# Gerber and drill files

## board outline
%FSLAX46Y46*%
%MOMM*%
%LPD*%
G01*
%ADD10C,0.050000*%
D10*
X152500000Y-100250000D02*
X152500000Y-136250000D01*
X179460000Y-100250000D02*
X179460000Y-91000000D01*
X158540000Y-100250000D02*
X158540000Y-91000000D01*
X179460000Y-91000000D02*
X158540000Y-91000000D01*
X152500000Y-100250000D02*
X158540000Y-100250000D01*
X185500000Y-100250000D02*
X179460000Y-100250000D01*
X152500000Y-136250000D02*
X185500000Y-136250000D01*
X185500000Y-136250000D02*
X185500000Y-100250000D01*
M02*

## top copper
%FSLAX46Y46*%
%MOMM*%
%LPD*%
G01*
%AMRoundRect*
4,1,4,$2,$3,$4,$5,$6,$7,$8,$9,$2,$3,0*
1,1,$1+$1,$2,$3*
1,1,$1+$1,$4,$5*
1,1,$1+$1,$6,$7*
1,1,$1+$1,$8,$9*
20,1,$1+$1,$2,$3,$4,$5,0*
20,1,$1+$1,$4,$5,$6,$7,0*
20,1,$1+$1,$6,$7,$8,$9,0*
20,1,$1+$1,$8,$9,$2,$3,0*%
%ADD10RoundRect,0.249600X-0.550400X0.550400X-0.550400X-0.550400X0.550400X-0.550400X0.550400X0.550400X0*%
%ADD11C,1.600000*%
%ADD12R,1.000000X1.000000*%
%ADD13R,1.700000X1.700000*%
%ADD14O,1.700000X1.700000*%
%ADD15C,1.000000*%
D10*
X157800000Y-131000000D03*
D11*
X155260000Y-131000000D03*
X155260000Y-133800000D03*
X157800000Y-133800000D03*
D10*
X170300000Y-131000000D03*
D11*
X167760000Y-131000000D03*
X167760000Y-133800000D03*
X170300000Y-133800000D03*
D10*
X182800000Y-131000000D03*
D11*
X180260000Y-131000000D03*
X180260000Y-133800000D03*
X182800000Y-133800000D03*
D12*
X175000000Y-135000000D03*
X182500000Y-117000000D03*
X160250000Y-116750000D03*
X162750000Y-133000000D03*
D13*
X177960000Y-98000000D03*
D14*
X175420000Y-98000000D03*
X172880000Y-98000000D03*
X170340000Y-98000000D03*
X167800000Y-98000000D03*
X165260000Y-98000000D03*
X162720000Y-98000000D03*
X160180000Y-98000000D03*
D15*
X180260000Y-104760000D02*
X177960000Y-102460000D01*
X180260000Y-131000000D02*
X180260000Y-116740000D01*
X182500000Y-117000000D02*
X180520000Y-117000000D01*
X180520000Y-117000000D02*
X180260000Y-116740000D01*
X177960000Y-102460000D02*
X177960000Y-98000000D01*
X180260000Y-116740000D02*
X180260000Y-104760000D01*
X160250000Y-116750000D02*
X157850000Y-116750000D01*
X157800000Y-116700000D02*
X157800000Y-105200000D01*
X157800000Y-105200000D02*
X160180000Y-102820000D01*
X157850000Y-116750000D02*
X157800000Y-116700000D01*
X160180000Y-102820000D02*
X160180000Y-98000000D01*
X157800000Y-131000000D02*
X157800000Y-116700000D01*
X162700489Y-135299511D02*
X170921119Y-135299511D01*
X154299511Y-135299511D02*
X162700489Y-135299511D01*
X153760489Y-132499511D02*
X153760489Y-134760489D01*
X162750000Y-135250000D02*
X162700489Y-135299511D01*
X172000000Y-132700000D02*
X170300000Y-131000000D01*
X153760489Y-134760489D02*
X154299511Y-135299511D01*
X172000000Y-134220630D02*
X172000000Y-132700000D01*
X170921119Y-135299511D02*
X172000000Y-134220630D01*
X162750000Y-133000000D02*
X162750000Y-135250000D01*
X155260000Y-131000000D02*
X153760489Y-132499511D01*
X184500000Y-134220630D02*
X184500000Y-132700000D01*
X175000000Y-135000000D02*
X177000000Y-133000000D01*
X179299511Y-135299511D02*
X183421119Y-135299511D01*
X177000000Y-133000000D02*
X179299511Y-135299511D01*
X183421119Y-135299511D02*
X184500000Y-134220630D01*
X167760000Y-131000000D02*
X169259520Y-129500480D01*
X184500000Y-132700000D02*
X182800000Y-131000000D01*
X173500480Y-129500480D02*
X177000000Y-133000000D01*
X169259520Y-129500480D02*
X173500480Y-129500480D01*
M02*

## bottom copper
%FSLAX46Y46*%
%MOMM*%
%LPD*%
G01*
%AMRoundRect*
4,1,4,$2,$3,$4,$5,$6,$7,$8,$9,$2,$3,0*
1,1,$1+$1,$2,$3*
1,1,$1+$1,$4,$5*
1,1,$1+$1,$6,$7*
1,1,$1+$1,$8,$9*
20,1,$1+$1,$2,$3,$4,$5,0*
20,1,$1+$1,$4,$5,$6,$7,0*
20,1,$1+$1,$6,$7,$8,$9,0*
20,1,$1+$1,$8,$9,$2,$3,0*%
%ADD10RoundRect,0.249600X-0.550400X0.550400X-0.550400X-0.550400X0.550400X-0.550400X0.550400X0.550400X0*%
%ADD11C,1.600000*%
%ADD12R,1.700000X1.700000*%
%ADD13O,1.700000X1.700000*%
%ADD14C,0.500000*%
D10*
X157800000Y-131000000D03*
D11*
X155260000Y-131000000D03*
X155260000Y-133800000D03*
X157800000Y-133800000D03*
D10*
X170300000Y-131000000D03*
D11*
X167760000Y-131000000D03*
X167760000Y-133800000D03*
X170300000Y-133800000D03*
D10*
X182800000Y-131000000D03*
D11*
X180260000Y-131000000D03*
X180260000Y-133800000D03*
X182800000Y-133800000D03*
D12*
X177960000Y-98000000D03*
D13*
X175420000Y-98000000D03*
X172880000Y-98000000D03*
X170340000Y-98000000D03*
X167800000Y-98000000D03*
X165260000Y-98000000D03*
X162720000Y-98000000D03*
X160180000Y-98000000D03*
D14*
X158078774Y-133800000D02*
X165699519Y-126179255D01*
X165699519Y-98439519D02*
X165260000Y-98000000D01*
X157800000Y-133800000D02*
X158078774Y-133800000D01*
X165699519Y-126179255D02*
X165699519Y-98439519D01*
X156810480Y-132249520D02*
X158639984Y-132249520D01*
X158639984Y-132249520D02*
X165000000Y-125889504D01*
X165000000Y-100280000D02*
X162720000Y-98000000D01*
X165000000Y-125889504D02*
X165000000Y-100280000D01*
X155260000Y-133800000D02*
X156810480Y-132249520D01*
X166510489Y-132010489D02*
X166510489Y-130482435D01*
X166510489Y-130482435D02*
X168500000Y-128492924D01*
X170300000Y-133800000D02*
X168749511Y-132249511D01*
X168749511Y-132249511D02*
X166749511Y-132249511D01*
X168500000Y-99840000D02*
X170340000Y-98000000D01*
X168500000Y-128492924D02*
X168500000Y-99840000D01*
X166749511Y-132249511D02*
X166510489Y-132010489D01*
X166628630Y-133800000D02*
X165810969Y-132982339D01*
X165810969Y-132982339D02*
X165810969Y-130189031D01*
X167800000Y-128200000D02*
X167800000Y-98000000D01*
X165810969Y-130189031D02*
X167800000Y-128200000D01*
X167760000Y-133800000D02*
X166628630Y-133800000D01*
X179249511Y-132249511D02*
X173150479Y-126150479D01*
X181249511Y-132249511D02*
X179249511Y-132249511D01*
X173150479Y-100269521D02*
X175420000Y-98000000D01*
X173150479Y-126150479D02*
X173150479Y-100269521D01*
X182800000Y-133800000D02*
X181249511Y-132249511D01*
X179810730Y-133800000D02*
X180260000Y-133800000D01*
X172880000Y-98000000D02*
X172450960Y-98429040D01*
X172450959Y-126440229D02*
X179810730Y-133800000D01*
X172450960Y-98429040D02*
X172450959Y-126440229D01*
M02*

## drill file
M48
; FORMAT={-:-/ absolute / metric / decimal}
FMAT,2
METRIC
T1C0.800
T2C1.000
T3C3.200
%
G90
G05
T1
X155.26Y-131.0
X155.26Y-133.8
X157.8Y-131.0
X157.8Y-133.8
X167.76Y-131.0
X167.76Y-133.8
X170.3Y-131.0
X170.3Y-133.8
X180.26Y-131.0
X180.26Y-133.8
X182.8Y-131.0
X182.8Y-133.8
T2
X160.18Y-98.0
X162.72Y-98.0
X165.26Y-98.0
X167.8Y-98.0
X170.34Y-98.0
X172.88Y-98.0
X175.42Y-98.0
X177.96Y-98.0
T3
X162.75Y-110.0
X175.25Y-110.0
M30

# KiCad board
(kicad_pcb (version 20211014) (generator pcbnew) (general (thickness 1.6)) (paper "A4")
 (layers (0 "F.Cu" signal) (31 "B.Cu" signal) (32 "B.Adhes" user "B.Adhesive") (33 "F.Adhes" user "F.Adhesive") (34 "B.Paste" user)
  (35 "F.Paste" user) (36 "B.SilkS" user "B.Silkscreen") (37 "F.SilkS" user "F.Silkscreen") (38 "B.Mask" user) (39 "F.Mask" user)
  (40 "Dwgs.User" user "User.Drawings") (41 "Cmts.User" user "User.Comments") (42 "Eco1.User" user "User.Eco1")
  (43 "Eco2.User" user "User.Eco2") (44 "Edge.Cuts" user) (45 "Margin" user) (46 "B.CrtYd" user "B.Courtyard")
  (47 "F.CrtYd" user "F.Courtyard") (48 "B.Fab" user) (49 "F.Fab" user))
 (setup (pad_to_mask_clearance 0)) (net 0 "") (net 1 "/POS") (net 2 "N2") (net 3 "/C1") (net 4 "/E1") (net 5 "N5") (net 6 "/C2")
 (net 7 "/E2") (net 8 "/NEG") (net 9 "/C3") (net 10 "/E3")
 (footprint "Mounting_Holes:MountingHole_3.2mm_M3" (layer "F.Cu") (at 162.75 110)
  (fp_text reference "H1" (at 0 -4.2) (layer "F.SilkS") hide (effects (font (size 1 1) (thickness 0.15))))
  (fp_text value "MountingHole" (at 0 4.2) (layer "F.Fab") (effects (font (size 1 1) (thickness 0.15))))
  (pad "" np_thru_hole circle locked (at 0 0) (size 3.2 3.2) (drill 3.2) (layers *.Cu *.Mask)))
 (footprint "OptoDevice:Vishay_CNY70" (layer "F.Cu") (at 157.8 131 -90)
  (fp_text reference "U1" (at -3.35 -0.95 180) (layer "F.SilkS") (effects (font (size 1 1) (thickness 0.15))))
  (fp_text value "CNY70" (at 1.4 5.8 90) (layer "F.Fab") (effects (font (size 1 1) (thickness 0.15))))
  (pad "1" thru_hole roundrect (at 0 0 270) (size 1.6 1.6) (drill 0.8) (layers *.Cu *.Mask) (roundrect_rratio 0.156) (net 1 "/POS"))
  (pad "2" thru_hole circle (at 0 2.54 270) (size 1.6 1.6) (drill 0.8) (layers *.Cu *.Mask) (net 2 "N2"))
  (pad "3" thru_hole circle (at 2.8 2.54 270) (size 1.6 1.6) (drill 0.8) (layers *.Cu *.Mask) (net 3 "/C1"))
  (pad "4" thru_hole circle (at 2.8 0 270) (size 1.6 1.6) (drill 0.8) (layers *.Cu *.Mask) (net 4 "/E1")))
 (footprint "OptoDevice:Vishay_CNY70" (layer "F.Cu") (at 170.3 131 -90)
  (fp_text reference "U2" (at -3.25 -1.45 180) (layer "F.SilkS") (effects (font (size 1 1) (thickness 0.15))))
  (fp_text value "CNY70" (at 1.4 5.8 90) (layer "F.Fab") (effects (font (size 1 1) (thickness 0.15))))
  (pad "1" thru_hole roundrect (at 0 0 270) (size 1.6 1.6) (drill 0.8) (layers *.Cu *.Mask) (roundrect_rratio 0.156) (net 2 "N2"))
  (pad "2" thru_hole circle (at 0 2.54 270) (size 1.6 1.6) (drill 0.8) (layers *.Cu *.Mask) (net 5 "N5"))
  (pad "3" thru_hole circle (at 2.8 2.54 270) (size 1.6 1.6) (drill 0.8) (layers *.Cu *.Mask) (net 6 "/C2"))
  (pad "4" thru_hole circle (at 2.8 0 270) (size 1.6 1.6) (drill 0.8) (layers *.Cu *.Mask) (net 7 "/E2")))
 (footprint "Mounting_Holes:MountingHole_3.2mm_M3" (layer "F.Cu") (at 175.25 110)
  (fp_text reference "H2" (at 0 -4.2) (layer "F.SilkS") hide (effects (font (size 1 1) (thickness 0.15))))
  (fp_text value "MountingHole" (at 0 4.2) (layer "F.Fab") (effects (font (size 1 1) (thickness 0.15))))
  (pad "" np_thru_hole circle locked (at 0 0) (size 3.2 3.2) (drill 3.2) (layers *.Cu *.Mask)))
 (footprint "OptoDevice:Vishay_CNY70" (layer "F.Cu") (at 182.8 131 -90)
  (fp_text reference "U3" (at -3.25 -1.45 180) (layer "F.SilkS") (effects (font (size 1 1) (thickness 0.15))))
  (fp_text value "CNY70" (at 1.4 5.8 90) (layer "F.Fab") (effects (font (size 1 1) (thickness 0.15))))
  (pad "1" thru_hole roundrect (at 0 0 270) (size 1.6 1.6) (drill 0.8) (layers *.Cu *.Mask) (roundrect_rratio 0.156) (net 5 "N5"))
  (pad "2" thru_hole circle (at 0 2.54 270) (size 1.6 1.6) (drill 0.8) (layers *.Cu *.Mask) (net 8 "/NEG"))
  (pad "3" thru_hole circle (at 2.8 2.54 270) (size 1.6 1.6) (drill 0.8) (layers *.Cu *.Mask) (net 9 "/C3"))
  (pad "4" thru_hole circle (at 2.8 0 270) (size 1.6 1.6) (drill 0.8) (layers *.Cu *.Mask) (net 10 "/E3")))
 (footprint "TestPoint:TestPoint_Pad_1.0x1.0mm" (layer "F.Cu") (at 175 135)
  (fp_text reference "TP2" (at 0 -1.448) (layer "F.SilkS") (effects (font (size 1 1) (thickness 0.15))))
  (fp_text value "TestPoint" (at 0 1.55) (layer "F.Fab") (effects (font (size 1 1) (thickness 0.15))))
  (pad "1" smd rect locked (at 0 0) (size 1 1) (layers "F.Cu" "F.Mask") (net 5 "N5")))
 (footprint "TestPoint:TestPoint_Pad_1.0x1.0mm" (layer "F.Cu") (at 182.5 117)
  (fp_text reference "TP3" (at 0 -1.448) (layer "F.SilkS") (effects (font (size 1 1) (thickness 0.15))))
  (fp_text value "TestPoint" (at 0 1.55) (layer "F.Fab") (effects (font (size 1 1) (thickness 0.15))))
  (pad "1" smd rect locked (at 0 0) (size 1 1) (layers "F.Cu" "F.Mask") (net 8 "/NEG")))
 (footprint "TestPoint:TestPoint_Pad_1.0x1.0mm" (layer "F.Cu") (at 160.25 116.75)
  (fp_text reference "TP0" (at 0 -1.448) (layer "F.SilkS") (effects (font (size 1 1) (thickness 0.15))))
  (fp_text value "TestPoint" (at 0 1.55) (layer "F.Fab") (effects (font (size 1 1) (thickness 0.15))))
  (pad "1" smd rect locked (at 0 0) (size 1 1) (layers "F.Cu" "F.Mask") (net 1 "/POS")))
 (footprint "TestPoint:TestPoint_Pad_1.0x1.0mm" (layer "F.Cu") (at 162.75 133)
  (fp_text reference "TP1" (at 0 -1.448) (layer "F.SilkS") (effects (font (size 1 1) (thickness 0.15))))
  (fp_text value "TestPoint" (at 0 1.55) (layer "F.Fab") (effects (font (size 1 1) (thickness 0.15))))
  (pad "1" smd rect locked (at 0 0) (size 1 1) (layers "F.Cu" "F.Mask") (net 2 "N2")))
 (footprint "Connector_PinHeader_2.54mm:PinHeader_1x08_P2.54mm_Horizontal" (layer "B.Cu") (at 177.96 98 90)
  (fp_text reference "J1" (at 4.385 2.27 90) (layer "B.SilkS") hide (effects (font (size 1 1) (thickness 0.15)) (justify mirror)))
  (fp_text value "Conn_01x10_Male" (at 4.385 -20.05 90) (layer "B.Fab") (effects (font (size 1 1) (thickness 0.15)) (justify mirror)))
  (pad "1" thru_hole rect (at 0 0 90) (size 1.7 1.7) (drill 1) (layers *.Cu *.Mask) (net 8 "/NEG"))
  (pad "2" thru_hole oval (at 0 -2.54 90) (size 1.7 1.7) (drill 1) (layers *.Cu *.Mask) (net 10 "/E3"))
  (pad "3" thru_hole oval (at 0 -5.08 90) (size 1.7 1.7) (drill 1) (layers *.Cu *.Mask) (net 9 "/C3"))
  (pad "4" thru_hole oval (at 0 -7.62 90) (size 1.7 1.7) (drill 1) (layers *.Cu *.Mask) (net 7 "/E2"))
  (pad "5" thru_hole oval (at 0 -10.16 90) (size 1.7 1.7) (drill 1) (layers *.Cu *.Mask) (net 6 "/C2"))
  (pad "6" thru_hole oval (at 0 -12.7 90) (size 1.7 1.7) (drill 1) (layers *.Cu *.Mask) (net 4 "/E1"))
  (pad "7" thru_hole oval (at 0 -15.24 90) (size 1.7 1.7) (drill 1) (layers *.Cu *.Mask) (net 3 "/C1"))
  (pad "8" thru_hole oval (at 0 -17.78 90) (size 1.7 1.7) (drill 1) (layers *.Cu *.Mask) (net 1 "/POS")))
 (gr_line (start 152.5 100.25) (end 152.5 136.25) (layer "Edge.Cuts") (width 0.05))
 (gr_line (start 179.46 100.25) (end 179.46 91) (layer "Edge.Cuts") (width 0.05))
 (gr_line (start 158.54 100.25) (end 158.54 91) (layer "Edge.Cuts") (width 0.05))
 (gr_line (start 179.46 91) (end 158.54 91) (layer "Edge.Cuts") (width 0.05))
 (gr_line (start 152.5 100.25) (end 158.54 100.25) (layer "Edge.Cuts") (width 0.05))
 (gr_line (start 185.5 100.25) (end 179.46 100.25) (layer "Edge.Cuts") (width 0.05))
 (gr_line (start 152.5 136.25) (end 185.5 136.25) (layer "Edge.Cuts") (width 0.05))
 (gr_line (start 185.5 136.25) (end 185.5 100.25) (layer "Edge.Cuts") (width 0.05))
 (segment (start 180.26 104.76) (end 177.96 102.46) (width 1) (layer "F.Cu") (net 8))
 (segment (start 180.26 131) (end 180.26 116.74) (width 1) (layer "F.Cu") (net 8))
 (segment (start 182.5 117) (end 180.52 117) (width 1) (layer "F.Cu") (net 8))
 (segment (start 180.52 117) (end 180.26 116.74) (width 1) (layer "F.Cu") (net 8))
 (segment (start 177.96 102.46) (end 177.96 98) (width 1) (layer "F.Cu") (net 8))
 (segment (start 180.26 116.74) (end 180.26 104.76) (width 1) (layer "F.Cu") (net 8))
 (segment (start 158.078774 133.8) (end 165.699519 126.179255) (width 0.5) (layer "B.Cu") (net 4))
 (segment (start 165.699519 98.439519) (end 165.26 98) (width 0.5) (layer "B.Cu") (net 4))
 (segment (start 157.8 133.8) (end 158.078774 133.8) (width 0.5) (layer "B.Cu") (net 4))
 (segment (start 165.699519 126.179255) (end 165.699519 98.439519) (width 0.5) (layer "B.Cu") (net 4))
 (segment (start 156.81048 132.24952) (end 158.639984 132.24952) (width 0.5) (layer "B.Cu") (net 3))
 (segment (start 158.639984 132.24952) (end 165 125.889504) (width 0.5) (layer "B.Cu") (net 3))
 (segment (start 165 100.28) (end 162.72 98) (width 0.5) (layer "B.Cu") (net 3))
 (segment (start 165 125.889504) (end 165 100.28) (width 0.5) (layer "B.Cu") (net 3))
 (segment (start 155.26 133.8) (end 156.81048 132.24952) (width 0.5) (layer "B.Cu") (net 3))
 (segment (start 160.25 116.75) (end 157.85 116.75) (width 1) (layer "F.Cu") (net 1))
 (segment (start 157.8 116.7) (end 157.8 105.2) (width 1) (layer "F.Cu") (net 1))
 (segment (start 157.8 105.2) (end 160.18 102.82) (width 1) (layer "F.Cu") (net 1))
 (segment (start 157.85 116.75) (end 157.8 116.7) (width 1) (layer "F.Cu") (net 1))
 (segment (start 160.18 102.82) (end 160.18 98) (width 1) (layer "F.Cu") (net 1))
 (segment (start 157.8 131) (end 157.8 116.7) (width 1) (layer "F.Cu") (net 1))
 (segment (start 162.700489 135.299511) (end 170.921119 135.299511) (width 1) (layer "F.Cu") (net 2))
 (segment (start 154.299511 135.299511) (end 162.700489 135.299511) (width 1) (layer "F.Cu") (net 2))
 (segment (start 153.760489 132.499511) (end 153.760489 134.760489) (width 1) (layer "F.Cu") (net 2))
 (segment (start 162.75 135.25) (end 162.700489 135.299511) (width 1) (layer "F.Cu") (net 2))
 (segment (start 172 132.7) (end 170.3 131) (width 1) (layer "F.Cu") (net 2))
 (segment (start 153.760489 134.760489) (end 154.299511 135.299511) (width 1) (layer "F.Cu") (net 2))
 (segment (start 172 134.22063) (end 172 132.7) (width 1) (layer "F.Cu") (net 2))
 (segment (start 170.921119 135.299511) (end 172 134.22063) (width 1) (layer "F.Cu") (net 2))
 (segment (start 162.75 133) (end 162.75 135.25) (width 1) (layer "F.Cu") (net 2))
 (segment (start 155.26 131) (end 153.760489 132.499511) (width 1) (layer "F.Cu") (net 2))
 (segment (start 166.510489 132.010489) (end 166.510489 130.482435) (width 0.5) (layer "B.Cu") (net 7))
 (segment (start 166.510489 130.482435) (end 168.5 128.492924) (width 0.5) (layer "B.Cu") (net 7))
 (segment (start 170.3 133.8) (end 168.749511 132.249511) (width 0.5) (layer "B.Cu") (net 7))
 (segment (start 168.749511 132.249511) (end 166.749511 132.249511) (width 0.5) (layer "B.Cu") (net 7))
 (segment (start 168.5 99.84) (end 170.34 98) (width 0.5) (layer "B.Cu") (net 7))
 (segment (start 168.5 128.492924) (end 168.5 99.84) (width 0.5) (layer "B.Cu") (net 7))
 (segment (start 166.749511 132.249511) (end 166.510489 132.010489) (width 0.5) (layer "B.Cu") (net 7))
 (segment (start 166.62863 133.8) (end 165.810969 132.982339) (width 0.5) (layer "B.Cu") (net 6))
 (segment (start 165.810969 132.982339) (end 165.810969 130.189031) (width 0.5) (layer "B.Cu") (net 6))
 (segment (start 167.8 128.2) (end 167.8 98) (width 0.5) (layer "B.Cu") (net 6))
 (segment (start 165.810969 130.189031) (end 167.8 128.2) (width 0.5) (layer "B.Cu") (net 6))
 (segment (start 167.76 133.8) (end 166.62863 133.8) (width 0.5) (layer "B.Cu") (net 6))
 (segment (start 179.249511 132.249511) (end 173.150479 126.150479) (width 0.5) (layer "B.Cu") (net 10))
 (segment (start 181.249511 132.249511) (end 179.249511 132.249511) (width 0.5) (layer "B.Cu") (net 10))
 (segment (start 173.150479 100.269521) (end 175.42 98) (width 0.5) (layer "B.Cu") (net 10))
 (segment (start 173.150479 126.150479) (end 173.150479 100.269521) (width 0.5) (layer "B.Cu") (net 10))
 (segment (start 182.8 133.8) (end 181.249511 132.249511) (width 0.5) (layer "B.Cu") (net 10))
 (segment (start 179.81073 133.8) (end 180.26 133.8) (width 0.5) (layer "B.Cu") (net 9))
 (segment (start 172.88 98) (end 172.45096 98.42904) (width 0.5) (layer "B.Cu") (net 9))
 (segment (start 172.450959 126.440229) (end 179.81073 133.8) (width 0.5) (layer "B.Cu") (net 9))
 (segment (start 172.45096 98.42904) (end 172.450959 126.440229) (width 0.5) (layer "B.Cu") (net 9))
 (segment (start 184.5 134.22063) (end 184.5 132.7) (width 1) (layer "F.Cu") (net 5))
 (segment (start 175 135) (end 177 133) (width 1) (layer "F.Cu") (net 5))
 (segment (start 179.299511 135.299511) (end 183.421119 135.299511) (width 1) (layer "F.Cu") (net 5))
 (segment (start 177 133) (end 179.299511 135.299511) (width 1) (layer "F.Cu") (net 5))
 (segment (start 183.421119 135.299511) (end 184.5 134.22063) (width 1) (layer "F.Cu") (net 5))
 (segment (start 167.76 131) (end 169.25952 129.50048) (width 1) (layer "F.Cu") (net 5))
 (segment (start 184.5 132.7) (end 182.8 131) (width 1) (layer "F.Cu") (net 5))
 (segment (start 173.50048 129.50048) (end 177 133) (width 1) (layer "F.Cu") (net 5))
 (segment (start 169.25952 129.50048) (end 173.50048 129.50048) (width 1) (layer "F.Cu") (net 5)))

